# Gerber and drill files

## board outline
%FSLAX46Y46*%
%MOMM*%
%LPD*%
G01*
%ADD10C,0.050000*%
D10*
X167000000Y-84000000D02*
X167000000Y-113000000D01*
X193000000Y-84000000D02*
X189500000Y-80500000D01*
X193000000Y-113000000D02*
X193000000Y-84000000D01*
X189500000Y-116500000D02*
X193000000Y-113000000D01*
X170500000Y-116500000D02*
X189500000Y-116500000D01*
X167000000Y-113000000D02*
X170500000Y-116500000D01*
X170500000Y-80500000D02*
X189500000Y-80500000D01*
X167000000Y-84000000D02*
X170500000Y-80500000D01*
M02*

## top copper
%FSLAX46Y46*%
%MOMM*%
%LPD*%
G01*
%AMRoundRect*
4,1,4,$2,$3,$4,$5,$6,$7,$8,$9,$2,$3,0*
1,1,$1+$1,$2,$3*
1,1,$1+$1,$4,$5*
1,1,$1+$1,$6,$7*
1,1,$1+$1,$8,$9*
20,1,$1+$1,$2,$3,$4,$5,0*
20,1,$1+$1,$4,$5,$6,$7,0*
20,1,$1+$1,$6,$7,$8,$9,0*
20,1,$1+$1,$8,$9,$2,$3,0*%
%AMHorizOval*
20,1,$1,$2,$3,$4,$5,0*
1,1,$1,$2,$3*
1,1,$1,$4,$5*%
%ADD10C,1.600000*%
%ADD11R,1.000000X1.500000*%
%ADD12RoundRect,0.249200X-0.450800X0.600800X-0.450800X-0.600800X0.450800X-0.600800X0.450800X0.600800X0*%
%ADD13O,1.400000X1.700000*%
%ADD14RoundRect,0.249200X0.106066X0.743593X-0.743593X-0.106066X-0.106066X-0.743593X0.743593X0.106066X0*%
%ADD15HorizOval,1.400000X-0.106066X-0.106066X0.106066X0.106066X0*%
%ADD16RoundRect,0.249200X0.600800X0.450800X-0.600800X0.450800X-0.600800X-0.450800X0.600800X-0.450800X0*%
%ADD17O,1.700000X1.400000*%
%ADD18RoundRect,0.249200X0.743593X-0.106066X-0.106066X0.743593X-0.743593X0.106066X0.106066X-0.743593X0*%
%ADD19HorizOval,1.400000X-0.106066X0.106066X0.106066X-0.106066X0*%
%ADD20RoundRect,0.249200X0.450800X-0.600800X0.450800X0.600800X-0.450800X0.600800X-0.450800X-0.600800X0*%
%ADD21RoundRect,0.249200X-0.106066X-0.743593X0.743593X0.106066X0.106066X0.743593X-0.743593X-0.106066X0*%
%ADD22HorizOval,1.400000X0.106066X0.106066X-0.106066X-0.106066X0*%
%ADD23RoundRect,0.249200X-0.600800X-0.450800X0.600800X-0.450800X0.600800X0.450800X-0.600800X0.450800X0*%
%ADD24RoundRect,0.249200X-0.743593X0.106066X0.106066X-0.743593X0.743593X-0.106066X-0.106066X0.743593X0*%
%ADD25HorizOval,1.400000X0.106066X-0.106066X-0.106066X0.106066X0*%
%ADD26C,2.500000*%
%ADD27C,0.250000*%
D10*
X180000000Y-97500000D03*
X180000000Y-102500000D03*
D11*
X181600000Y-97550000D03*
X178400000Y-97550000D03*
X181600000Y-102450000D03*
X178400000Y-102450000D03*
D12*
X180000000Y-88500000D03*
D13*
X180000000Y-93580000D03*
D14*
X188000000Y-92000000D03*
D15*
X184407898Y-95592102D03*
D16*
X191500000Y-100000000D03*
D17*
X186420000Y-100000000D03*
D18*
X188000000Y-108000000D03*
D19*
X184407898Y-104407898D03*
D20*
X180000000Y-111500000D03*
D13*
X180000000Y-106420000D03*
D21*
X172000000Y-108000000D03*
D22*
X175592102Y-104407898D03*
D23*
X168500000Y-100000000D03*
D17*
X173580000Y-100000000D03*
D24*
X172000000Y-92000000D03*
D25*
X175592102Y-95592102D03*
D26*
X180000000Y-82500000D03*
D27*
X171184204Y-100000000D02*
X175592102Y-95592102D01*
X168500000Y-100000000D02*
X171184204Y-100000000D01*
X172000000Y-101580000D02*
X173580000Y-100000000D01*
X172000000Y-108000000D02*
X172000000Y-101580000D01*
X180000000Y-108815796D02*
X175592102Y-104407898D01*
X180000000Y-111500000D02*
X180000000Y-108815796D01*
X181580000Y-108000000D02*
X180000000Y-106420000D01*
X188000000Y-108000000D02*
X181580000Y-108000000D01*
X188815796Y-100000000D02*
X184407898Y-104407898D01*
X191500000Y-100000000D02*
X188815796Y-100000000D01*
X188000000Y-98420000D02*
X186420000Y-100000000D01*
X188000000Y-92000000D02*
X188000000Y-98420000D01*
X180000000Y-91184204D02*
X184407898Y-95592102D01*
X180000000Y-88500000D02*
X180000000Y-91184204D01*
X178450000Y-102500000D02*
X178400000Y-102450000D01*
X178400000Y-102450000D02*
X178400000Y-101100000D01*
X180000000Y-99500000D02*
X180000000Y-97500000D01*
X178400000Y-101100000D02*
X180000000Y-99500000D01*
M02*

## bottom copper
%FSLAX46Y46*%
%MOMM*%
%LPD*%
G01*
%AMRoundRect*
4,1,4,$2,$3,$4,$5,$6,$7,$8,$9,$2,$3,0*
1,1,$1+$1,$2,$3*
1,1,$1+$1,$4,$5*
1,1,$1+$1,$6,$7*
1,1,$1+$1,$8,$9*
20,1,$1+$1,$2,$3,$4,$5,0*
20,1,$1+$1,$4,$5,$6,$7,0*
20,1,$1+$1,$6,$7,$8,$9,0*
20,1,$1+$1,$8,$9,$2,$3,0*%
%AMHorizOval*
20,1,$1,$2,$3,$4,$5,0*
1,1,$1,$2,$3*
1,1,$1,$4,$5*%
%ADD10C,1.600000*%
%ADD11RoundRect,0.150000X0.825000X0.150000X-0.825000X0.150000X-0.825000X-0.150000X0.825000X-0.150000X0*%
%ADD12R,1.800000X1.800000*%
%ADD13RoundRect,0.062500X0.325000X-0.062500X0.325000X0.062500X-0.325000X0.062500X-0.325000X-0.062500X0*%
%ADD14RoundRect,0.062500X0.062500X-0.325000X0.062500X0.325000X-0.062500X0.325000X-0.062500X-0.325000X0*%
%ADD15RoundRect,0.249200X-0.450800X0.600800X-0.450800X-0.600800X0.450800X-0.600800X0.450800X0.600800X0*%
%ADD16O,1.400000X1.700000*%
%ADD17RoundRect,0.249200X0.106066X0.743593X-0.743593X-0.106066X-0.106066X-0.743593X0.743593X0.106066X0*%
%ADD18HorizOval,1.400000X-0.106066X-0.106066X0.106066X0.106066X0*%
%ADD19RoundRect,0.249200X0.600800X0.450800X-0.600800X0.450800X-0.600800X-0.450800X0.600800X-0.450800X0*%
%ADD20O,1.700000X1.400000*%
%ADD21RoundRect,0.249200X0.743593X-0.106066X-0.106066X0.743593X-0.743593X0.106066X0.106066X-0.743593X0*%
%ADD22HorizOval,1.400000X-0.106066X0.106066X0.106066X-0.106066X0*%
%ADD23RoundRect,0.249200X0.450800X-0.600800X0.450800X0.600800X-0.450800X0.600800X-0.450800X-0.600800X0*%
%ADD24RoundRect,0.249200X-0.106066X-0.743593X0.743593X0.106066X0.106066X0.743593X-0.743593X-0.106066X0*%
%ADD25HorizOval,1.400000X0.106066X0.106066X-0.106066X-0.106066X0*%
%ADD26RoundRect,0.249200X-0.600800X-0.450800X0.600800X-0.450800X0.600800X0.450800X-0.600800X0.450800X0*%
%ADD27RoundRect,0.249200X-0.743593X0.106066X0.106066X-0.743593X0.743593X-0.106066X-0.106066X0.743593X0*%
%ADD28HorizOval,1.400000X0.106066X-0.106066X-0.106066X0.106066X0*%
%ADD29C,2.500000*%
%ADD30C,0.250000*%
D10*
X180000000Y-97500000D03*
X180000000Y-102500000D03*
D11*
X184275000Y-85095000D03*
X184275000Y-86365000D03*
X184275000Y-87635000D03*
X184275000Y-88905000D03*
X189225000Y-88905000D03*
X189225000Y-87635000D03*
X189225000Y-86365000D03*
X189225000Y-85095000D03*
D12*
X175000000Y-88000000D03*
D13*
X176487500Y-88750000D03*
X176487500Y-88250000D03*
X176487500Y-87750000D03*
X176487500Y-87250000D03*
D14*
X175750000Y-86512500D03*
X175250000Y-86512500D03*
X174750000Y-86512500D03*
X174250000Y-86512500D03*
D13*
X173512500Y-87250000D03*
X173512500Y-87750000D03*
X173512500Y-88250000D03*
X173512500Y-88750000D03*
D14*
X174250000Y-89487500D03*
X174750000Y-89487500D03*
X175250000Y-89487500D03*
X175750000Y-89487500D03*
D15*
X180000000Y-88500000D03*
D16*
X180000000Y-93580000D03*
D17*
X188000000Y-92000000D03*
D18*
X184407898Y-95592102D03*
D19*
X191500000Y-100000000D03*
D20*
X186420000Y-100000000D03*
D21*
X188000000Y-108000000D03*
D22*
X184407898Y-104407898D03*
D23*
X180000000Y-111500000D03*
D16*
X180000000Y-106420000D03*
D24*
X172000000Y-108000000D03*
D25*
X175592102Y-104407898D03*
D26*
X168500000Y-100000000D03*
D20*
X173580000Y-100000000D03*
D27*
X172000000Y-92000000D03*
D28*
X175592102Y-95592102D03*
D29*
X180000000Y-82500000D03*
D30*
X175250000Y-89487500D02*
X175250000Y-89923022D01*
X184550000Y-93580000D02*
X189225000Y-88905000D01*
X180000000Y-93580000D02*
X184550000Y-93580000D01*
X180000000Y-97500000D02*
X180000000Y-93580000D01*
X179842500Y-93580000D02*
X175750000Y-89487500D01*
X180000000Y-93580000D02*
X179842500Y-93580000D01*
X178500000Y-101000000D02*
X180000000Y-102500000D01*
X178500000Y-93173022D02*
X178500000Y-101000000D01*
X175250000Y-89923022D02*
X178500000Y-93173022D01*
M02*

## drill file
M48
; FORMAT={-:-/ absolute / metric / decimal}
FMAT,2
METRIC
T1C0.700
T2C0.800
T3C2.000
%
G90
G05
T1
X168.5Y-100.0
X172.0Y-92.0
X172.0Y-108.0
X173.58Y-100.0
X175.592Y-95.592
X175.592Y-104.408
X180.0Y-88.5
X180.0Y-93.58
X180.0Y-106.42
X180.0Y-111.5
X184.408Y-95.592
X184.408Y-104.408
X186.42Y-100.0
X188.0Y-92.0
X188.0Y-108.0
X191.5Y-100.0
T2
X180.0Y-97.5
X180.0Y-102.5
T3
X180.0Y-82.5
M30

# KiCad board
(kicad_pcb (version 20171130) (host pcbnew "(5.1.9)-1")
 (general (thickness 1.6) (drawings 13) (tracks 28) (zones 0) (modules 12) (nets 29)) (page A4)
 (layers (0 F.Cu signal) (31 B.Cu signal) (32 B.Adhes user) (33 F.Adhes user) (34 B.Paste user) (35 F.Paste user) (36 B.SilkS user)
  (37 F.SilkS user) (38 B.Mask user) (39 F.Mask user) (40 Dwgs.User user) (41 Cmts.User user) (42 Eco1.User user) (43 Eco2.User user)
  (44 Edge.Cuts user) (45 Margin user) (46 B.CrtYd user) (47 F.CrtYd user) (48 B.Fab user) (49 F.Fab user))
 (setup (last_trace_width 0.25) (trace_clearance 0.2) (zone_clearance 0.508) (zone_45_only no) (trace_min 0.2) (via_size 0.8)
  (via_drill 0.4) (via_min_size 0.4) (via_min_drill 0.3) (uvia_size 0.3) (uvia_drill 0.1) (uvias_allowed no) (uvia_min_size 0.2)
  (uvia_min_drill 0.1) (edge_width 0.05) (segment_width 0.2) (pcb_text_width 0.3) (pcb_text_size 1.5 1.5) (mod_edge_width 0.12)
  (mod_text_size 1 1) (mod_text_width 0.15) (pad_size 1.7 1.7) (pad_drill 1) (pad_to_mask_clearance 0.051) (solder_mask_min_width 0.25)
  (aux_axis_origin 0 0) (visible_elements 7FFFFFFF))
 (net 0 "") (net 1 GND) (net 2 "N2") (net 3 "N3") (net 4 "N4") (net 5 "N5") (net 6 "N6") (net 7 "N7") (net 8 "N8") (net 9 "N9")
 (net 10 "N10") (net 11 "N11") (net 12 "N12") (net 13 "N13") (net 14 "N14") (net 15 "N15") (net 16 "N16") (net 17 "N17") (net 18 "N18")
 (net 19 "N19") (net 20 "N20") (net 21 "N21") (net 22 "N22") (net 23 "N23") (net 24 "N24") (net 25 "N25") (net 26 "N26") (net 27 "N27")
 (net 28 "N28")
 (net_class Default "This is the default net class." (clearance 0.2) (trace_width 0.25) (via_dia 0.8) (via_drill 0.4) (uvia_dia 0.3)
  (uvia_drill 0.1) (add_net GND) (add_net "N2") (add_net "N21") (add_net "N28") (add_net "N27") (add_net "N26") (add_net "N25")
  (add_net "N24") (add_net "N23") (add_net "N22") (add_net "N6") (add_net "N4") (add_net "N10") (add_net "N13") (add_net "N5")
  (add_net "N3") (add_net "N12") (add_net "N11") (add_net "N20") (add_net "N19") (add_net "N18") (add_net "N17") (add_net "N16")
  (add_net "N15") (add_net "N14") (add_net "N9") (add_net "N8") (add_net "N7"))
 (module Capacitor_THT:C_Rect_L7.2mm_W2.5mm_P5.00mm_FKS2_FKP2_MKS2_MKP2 (layer B.Cu) (at 180 102.5 90)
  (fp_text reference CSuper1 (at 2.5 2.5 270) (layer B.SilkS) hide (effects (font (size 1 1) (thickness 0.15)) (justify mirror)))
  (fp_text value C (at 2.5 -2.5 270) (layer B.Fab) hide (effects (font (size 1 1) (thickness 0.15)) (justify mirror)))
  (pad 2 thru_hole circle (at 5 0 90) (size 1.6 1.6) (drill 0.8) (layers *.Cu *.Mask) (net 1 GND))
  (pad 1 thru_hole circle (at 0 0 90) (size 1.6 1.6) (drill 0.8) (layers *.Cu *.Mask) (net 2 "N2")))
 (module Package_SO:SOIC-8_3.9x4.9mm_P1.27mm (layer B.Cu) (at 186.75 87 180)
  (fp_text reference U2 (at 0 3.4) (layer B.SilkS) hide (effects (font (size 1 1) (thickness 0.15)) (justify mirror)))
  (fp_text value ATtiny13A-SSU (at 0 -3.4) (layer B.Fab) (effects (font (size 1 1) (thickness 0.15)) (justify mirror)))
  (pad 8 smd roundrect (at 2.475 1.905 180) (size 1.95 0.6) (layers B.Cu B.Paste B.Mask) (roundrect_rratio 0.25) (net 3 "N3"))
  (pad 7 smd roundrect (at 2.475 0.635 180) (size 1.95 0.6) (layers B.Cu B.Paste B.Mask) (roundrect_rratio 0.25) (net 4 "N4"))
  (pad 6 smd roundrect (at 2.475 -0.635 180) (size 1.95 0.6) (layers B.Cu B.Paste B.Mask) (roundrect_rratio 0.25) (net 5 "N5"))
  (pad 5 smd roundrect (at 2.475 -1.905 180) (size 1.95 0.6) (layers B.Cu B.Paste B.Mask) (roundrect_rratio 0.25) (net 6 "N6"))
  (pad 4 smd roundrect (at -2.475 -1.905 180) (size 1.95 0.6) (layers B.Cu B.Paste B.Mask) (roundrect_rratio 0.25) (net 1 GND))
  (pad 3 smd roundrect (at -2.475 -0.635 180) (size 1.95 0.6) (layers B.Cu B.Paste B.Mask) (roundrect_rratio 0.25) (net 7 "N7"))
  (pad 2 smd roundrect (at -2.475 0.635 180) (size 1.95 0.6) (layers B.Cu B.Paste B.Mask) (roundrect_rratio 0.25) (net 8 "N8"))
  (pad 1 smd roundrect (at -2.475 1.905 180) (size 1.95 0.6) (layers B.Cu B.Paste B.Mask) (roundrect_rratio 0.25) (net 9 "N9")))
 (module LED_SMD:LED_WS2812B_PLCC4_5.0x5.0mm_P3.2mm (layer F.Cu) (at 180 100 90)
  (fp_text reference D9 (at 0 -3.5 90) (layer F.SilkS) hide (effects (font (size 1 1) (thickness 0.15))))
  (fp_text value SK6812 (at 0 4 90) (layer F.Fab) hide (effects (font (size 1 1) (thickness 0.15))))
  (pad 3 smd rect (at 2.45 1.6 90) (size 1.5 1) (layers F.Cu F.Paste F.Mask) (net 4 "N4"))
  (pad 4 smd rect (at 2.45 -1.6 90) (size 1.5 1) (layers F.Cu F.Paste F.Mask) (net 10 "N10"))
  (pad 2 smd rect (at -2.45 1.6 90) (size 1.5 1) (layers F.Cu F.Paste F.Mask) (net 6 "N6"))
  (pad 1 smd rect (at -2.45 -1.6 90) (size 1.5 1) (layers F.Cu F.Paste F.Mask) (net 1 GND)))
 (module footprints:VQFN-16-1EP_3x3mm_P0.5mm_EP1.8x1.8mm (layer B.Cu) (at 175 88 90)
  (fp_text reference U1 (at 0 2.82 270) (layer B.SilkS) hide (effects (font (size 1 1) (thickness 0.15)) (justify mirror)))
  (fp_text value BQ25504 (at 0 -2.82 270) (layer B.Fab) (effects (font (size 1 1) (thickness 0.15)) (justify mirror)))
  (pad "" smd roundrect (at 0.45 -0.45 90) (size 0.73 0.73) (layers B.Paste) (roundrect_rratio 0.25))
  (pad "" smd roundrect (at 0.45 0.45 90) (size 0.73 0.73) (layers B.Paste) (roundrect_rratio 0.25))
  (pad "" smd roundrect (at -0.45 -0.45 90) (size 0.73 0.73) (layers B.Paste) (roundrect_rratio 0.25))
  (pad "" smd roundrect (at -0.45 0.45 90) (size 0.73 0.73) (layers B.Paste) (roundrect_rratio 0.25))
  (pad 17 smd rect (at 0 0 90) (size 1.8 1.8) (layers B.Cu B.Mask) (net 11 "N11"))
  (pad 16 smd roundrect (at -0.75 1.4875 90) (size 0.25 0.775) (layers B.Cu B.Paste B.Mask) (roundrect_rratio 0.25) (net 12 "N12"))
  (pad 15 smd roundrect (at -0.25 1.4875 90) (size 0.25 0.775) (layers B.Cu B.Paste B.Mask) (roundrect_rratio 0.25) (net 3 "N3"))
  (pad 14 smd roundrect (at 0.25 1.4875 90) (size 0.25 0.775) (layers B.Cu B.Paste B.Mask) (roundrect_rratio 0.25) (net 2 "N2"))
  (pad 13 smd roundrect (at 0.75 1.4875 90) (size 0.25 0.775) (layers B.Cu B.Paste B.Mask) (roundrect_rratio 0.25) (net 1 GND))
  (pad 12 smd roundrect (at 1.4875 0.75 90) (size 0.775 0.25) (layers B.Cu B.Paste B.Mask) (roundrect_rratio 0.25) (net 1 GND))
  (pad 11 smd roundrect (at 1.4875 0.25 90) (size 0.775 0.25) (layers B.Cu B.Paste B.Mask) (roundrect_rratio 0.25) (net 5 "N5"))
  (pad 10 smd roundrect (at 1.4875 -0.25 90) (size 0.775 0.25) (layers B.Cu B.Paste B.Mask) (roundrect_rratio 0.25) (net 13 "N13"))
  (pad 9 smd roundrect (at 1.4875 -0.75 90) (size 0.775 0.25) (layers B.Cu B.Paste B.Mask) (roundrect_rratio 0.25) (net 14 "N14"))
  (pad 8 smd roundrect (at 0.75 -1.4875 90) (size 0.25 0.775) (layers B.Cu B.Paste B.Mask) (roundrect_rratio 0.25) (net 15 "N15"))
  (pad 7 smd roundrect (at 0.25 -1.4875 90) (size 0.25 0.775) (layers B.Cu B.Paste B.Mask) (roundrect_rratio 0.25) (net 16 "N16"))
  (pad 6 smd roundrect (at -0.25 -1.4875 90) (size 0.25 0.775) (layers B.Cu B.Paste B.Mask) (roundrect_rratio 0.25) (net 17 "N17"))
  (pad 5 smd roundrect (at -0.75 -1.4875 90) (size 0.25 0.775) (layers B.Cu B.Paste B.Mask) (roundrect_rratio 0.25) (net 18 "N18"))
  (pad 4 smd roundrect (at -1.4875 -0.75 90) (size 0.775 0.25) (layers B.Cu B.Paste B.Mask) (roundrect_rratio 0.25) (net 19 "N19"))
  (pad 3 smd roundrect (at -1.4875 -0.25 90) (size 0.775 0.25) (layers B.Cu B.Paste B.Mask) (roundrect_rratio 0.25) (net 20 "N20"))
  (pad 2 smd roundrect (at -1.4875 0.25 90) (size 0.775 0.25) (layers B.Cu B.Paste B.Mask) (roundrect_rratio 0.25) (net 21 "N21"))
  (pad 1 smd roundrect (at -1.4875 0.75 90) (size 0.775 0.25) (layers B.Cu B.Paste B.Mask) (roundrect_rratio 0.25) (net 1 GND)))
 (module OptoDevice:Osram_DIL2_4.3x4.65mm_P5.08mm (layer F.Cu) (at 180 88.5 270)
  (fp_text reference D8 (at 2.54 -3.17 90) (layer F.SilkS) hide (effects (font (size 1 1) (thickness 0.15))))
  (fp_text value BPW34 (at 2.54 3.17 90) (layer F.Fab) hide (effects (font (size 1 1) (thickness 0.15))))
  (pad 1 thru_hole roundrect (at 0 0 270) (size 1.7 1.4) (drill 0.7) (layers *.Cu *.Mask) (roundrect_rratio 0.178) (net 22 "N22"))
  (pad 2 thru_hole oval (at 5.08 0 270) (size 1.7 1.4) (drill 0.7) (layers *.Cu *.Mask) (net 1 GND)))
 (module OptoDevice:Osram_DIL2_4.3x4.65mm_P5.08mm (layer F.Cu) (at 188 92 225)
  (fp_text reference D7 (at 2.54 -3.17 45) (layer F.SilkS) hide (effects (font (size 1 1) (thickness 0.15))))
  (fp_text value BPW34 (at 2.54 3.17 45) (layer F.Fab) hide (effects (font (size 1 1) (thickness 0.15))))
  (pad 1 thru_hole roundrect (at 0 0 225) (size 1.7 1.4) (drill 0.7) (layers *.Cu *.Mask) (roundrect_rratio 0.178) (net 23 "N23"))
  (pad 2 thru_hole oval (at 5.08 0 225) (size 1.7 1.4) (drill 0.7) (layers *.Cu *.Mask) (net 22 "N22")))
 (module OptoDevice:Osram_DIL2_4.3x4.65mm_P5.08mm (layer F.Cu) (at 191.5 100 180)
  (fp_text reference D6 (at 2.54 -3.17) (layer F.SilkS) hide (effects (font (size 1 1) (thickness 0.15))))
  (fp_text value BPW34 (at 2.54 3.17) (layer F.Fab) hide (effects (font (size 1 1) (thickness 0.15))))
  (pad 1 thru_hole roundrect (at 0 0 180) (size 1.7 1.4) (drill 0.7) (layers *.Cu *.Mask) (roundrect_rratio 0.178) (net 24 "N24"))
  (pad 2 thru_hole oval (at 5.08 0 180) (size 1.7 1.4) (drill 0.7) (layers *.Cu *.Mask) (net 23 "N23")))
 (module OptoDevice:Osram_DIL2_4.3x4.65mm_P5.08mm (layer F.Cu) (at 188 108 135)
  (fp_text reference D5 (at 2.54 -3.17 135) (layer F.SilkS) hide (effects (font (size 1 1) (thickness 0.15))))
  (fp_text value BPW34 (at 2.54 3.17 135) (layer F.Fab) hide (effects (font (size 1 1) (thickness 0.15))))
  (pad 1 thru_hole roundrect (at 0 0 135) (size 1.7 1.4) (drill 0.7) (layers *.Cu *.Mask) (roundrect_rratio 0.178) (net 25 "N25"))
  (pad 2 thru_hole oval (at 5.08 0 135) (size 1.7 1.4) (drill 0.7) (layers *.Cu *.Mask) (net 24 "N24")))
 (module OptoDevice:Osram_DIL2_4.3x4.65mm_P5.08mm (layer F.Cu) (at 180 111.5 90)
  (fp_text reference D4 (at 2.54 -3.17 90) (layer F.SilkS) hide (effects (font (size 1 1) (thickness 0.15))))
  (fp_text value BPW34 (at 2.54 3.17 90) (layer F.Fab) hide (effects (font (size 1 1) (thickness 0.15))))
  (pad 1 thru_hole roundrect (at 0 0 90) (size 1.7 1.4) (drill 0.7) (layers *.Cu *.Mask) (roundrect_rratio 0.178) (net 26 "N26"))
  (pad 2 thru_hole oval (at 5.08 0 90) (size 1.7 1.4) (drill 0.7) (layers *.Cu *.Mask) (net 25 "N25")))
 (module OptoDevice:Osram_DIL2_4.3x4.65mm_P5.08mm (layer F.Cu) (at 172 108 45)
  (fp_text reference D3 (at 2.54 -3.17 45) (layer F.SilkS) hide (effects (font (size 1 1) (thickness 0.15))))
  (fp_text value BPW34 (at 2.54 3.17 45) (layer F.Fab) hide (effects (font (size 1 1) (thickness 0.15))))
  (pad 1 thru_hole roundrect (at 0 0 45) (size 1.7 1.4) (drill 0.7) (layers *.Cu *.Mask) (roundrect_rratio 0.178) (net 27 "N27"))
  (pad 2 thru_hole oval (at 5.08 0 45) (size 1.7 1.4) (drill 0.7) (layers *.Cu *.Mask) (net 26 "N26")))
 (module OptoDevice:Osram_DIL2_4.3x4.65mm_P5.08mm (layer F.Cu) (at 168.5 100)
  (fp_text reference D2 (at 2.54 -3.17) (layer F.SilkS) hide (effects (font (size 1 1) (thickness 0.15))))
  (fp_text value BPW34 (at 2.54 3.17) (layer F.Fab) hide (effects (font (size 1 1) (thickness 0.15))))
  (pad 1 thru_hole roundrect (at 0 0) (size 1.7 1.4) (drill 0.7) (layers *.Cu *.Mask) (roundrect_rratio 0.178) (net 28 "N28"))
  (pad 2 thru_hole oval (at 5.08 0) (size 1.7 1.4) (drill 0.7) (layers *.Cu *.Mask) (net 27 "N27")))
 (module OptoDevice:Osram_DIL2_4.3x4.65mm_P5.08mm (layer F.Cu) (at 172 92 315)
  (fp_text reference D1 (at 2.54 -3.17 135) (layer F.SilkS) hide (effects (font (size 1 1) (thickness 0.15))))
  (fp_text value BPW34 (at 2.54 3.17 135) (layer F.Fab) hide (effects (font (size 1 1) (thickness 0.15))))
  (pad 1 thru_hole roundrect (at 0 0 315) (size 1.7 1.4) (drill 0.7) (layers *.Cu *.Mask) (roundrect_rratio 0.178) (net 21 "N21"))
  (pad 2 thru_hole oval (at 5.08 0 315) (size 1.7 1.4) (drill 0.7) (layers *.Cu *.Mask) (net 28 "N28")))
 (gr_line (start 167 84) (end 167 113) (layer Edge.Cuts) (width 0.05))
 (gr_line (start 193 84) (end 189.5 80.5) (layer Edge.Cuts) (width 0.05))
 (gr_line (start 193 113) (end 193 84) (layer Edge.Cuts) (width 0.05))
 (gr_line (start 189.5 116.5) (end 193 113) (layer Edge.Cuts) (width 0.05))
 (gr_line (start 170.5 116.5) (end 189.5 116.5) (layer Edge.Cuts) (width 0.05))
 (gr_line (start 167 113) (end 170.5 116.5) (layer Edge.Cuts) (width 0.05))
 (gr_line (start 170.5 80.5) (end 189.5 80.5) (layer Edge.Cuts) (width 0.05))
 (gr_line (start 167 84) (end 170.5 80.5) (layer Edge.Cuts) (width 0.05))
 (via (at 180 82.5) (size 2.5) (drill 2) (layers F.Cu B.Cu) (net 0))
 (segment (start 171.184204 100) (end 175.592102 95.592102) (width 0.25) (layer F.Cu) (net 28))
 (segment (start 168.5 100) (end 171.184204 100) (width 0.25) (layer F.Cu) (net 28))
 (segment (start 172 101.58) (end 173.58 100) (width 0.25) (layer F.Cu) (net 27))
 (segment (start 172 108) (end 172 101.58) (width 0.25) (layer F.Cu) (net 27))
 (segment (start 180 108.815796) (end 175.592102 104.407898) (width 0.25) (layer F.Cu) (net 26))
 (segment (start 180 111.5) (end 180 108.815796) (width 0.25) (layer F.Cu) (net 26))
 (segment (start 181.58 108) (end 180 106.42) (width 0.25) (layer F.Cu) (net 25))
 (segment (start 188 108) (end 181.58 108) (width 0.25) (layer F.Cu) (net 25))
 (segment (start 188.815796 100) (end 184.407898 104.407898) (width 0.25) (layer F.Cu) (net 24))
 (segment (start 191.5 100) (end 188.815796 100) (width 0.25) (layer F.Cu) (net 24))
 (segment (start 188 98.42) (end 186.42 100) (width 0.25) (layer F.Cu) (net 23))
 (segment (start 188 92) (end 188 98.42) (width 0.25) (layer F.Cu) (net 23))
 (segment (start 180 91.184204) (end 184.407898 95.592102) (width 0.25) (layer F.Cu) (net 22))
 (segment (start 180 88.5) (end 180 91.184204) (width 0.25) (layer F.Cu) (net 22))
 (segment (start 175.25 89.4875) (end 175.25 89.923022) (width 0.25) (layer B.Cu) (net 2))
 (segment (start 178.45 102.5) (end 178.4 102.45) (width 0.25) (layer F.Cu) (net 1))
 (segment (start 178.4 102.45) (end 178.4 101.1) (width 0.25) (layer F.Cu) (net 1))
 (segment (start 180 99.5) (end 180 97.5) (width 0.25) (layer F.Cu) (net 1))
 (segment (start 178.4 101.1) (end 180 99.5) (width 0.25) (layer F.Cu) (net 1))
 (segment (start 184.55 93.58) (end 189.225 88.905) (width 0.25) (layer B.Cu) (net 1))
 (segment (start 180 93.58) (end 184.55 93.58) (width 0.25) (layer B.Cu) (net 1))
 (segment (start 180 97.5) (end 180 93.58) (width 0.25) (layer B.Cu) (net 1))
 (segment (start 179.8425 93.58) (end 175.75 89.4875) (width 0.25) (layer B.Cu) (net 1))
 (segment (start 180 93.58) (end 179.8425 93.58) (width 0.25) (layer B.Cu) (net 1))
 (segment (start 178.5 101) (end 180 102.5) (width 0.25) (layer B.Cu) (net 2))
 (segment (start 178.5 93.173022) (end 178.5 101) (width 0.25) (layer B.Cu) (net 2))
 (segment (start 175.25 89.923022) (end 178.5 93.173022) (width 0.25) (layer B.Cu) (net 2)))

